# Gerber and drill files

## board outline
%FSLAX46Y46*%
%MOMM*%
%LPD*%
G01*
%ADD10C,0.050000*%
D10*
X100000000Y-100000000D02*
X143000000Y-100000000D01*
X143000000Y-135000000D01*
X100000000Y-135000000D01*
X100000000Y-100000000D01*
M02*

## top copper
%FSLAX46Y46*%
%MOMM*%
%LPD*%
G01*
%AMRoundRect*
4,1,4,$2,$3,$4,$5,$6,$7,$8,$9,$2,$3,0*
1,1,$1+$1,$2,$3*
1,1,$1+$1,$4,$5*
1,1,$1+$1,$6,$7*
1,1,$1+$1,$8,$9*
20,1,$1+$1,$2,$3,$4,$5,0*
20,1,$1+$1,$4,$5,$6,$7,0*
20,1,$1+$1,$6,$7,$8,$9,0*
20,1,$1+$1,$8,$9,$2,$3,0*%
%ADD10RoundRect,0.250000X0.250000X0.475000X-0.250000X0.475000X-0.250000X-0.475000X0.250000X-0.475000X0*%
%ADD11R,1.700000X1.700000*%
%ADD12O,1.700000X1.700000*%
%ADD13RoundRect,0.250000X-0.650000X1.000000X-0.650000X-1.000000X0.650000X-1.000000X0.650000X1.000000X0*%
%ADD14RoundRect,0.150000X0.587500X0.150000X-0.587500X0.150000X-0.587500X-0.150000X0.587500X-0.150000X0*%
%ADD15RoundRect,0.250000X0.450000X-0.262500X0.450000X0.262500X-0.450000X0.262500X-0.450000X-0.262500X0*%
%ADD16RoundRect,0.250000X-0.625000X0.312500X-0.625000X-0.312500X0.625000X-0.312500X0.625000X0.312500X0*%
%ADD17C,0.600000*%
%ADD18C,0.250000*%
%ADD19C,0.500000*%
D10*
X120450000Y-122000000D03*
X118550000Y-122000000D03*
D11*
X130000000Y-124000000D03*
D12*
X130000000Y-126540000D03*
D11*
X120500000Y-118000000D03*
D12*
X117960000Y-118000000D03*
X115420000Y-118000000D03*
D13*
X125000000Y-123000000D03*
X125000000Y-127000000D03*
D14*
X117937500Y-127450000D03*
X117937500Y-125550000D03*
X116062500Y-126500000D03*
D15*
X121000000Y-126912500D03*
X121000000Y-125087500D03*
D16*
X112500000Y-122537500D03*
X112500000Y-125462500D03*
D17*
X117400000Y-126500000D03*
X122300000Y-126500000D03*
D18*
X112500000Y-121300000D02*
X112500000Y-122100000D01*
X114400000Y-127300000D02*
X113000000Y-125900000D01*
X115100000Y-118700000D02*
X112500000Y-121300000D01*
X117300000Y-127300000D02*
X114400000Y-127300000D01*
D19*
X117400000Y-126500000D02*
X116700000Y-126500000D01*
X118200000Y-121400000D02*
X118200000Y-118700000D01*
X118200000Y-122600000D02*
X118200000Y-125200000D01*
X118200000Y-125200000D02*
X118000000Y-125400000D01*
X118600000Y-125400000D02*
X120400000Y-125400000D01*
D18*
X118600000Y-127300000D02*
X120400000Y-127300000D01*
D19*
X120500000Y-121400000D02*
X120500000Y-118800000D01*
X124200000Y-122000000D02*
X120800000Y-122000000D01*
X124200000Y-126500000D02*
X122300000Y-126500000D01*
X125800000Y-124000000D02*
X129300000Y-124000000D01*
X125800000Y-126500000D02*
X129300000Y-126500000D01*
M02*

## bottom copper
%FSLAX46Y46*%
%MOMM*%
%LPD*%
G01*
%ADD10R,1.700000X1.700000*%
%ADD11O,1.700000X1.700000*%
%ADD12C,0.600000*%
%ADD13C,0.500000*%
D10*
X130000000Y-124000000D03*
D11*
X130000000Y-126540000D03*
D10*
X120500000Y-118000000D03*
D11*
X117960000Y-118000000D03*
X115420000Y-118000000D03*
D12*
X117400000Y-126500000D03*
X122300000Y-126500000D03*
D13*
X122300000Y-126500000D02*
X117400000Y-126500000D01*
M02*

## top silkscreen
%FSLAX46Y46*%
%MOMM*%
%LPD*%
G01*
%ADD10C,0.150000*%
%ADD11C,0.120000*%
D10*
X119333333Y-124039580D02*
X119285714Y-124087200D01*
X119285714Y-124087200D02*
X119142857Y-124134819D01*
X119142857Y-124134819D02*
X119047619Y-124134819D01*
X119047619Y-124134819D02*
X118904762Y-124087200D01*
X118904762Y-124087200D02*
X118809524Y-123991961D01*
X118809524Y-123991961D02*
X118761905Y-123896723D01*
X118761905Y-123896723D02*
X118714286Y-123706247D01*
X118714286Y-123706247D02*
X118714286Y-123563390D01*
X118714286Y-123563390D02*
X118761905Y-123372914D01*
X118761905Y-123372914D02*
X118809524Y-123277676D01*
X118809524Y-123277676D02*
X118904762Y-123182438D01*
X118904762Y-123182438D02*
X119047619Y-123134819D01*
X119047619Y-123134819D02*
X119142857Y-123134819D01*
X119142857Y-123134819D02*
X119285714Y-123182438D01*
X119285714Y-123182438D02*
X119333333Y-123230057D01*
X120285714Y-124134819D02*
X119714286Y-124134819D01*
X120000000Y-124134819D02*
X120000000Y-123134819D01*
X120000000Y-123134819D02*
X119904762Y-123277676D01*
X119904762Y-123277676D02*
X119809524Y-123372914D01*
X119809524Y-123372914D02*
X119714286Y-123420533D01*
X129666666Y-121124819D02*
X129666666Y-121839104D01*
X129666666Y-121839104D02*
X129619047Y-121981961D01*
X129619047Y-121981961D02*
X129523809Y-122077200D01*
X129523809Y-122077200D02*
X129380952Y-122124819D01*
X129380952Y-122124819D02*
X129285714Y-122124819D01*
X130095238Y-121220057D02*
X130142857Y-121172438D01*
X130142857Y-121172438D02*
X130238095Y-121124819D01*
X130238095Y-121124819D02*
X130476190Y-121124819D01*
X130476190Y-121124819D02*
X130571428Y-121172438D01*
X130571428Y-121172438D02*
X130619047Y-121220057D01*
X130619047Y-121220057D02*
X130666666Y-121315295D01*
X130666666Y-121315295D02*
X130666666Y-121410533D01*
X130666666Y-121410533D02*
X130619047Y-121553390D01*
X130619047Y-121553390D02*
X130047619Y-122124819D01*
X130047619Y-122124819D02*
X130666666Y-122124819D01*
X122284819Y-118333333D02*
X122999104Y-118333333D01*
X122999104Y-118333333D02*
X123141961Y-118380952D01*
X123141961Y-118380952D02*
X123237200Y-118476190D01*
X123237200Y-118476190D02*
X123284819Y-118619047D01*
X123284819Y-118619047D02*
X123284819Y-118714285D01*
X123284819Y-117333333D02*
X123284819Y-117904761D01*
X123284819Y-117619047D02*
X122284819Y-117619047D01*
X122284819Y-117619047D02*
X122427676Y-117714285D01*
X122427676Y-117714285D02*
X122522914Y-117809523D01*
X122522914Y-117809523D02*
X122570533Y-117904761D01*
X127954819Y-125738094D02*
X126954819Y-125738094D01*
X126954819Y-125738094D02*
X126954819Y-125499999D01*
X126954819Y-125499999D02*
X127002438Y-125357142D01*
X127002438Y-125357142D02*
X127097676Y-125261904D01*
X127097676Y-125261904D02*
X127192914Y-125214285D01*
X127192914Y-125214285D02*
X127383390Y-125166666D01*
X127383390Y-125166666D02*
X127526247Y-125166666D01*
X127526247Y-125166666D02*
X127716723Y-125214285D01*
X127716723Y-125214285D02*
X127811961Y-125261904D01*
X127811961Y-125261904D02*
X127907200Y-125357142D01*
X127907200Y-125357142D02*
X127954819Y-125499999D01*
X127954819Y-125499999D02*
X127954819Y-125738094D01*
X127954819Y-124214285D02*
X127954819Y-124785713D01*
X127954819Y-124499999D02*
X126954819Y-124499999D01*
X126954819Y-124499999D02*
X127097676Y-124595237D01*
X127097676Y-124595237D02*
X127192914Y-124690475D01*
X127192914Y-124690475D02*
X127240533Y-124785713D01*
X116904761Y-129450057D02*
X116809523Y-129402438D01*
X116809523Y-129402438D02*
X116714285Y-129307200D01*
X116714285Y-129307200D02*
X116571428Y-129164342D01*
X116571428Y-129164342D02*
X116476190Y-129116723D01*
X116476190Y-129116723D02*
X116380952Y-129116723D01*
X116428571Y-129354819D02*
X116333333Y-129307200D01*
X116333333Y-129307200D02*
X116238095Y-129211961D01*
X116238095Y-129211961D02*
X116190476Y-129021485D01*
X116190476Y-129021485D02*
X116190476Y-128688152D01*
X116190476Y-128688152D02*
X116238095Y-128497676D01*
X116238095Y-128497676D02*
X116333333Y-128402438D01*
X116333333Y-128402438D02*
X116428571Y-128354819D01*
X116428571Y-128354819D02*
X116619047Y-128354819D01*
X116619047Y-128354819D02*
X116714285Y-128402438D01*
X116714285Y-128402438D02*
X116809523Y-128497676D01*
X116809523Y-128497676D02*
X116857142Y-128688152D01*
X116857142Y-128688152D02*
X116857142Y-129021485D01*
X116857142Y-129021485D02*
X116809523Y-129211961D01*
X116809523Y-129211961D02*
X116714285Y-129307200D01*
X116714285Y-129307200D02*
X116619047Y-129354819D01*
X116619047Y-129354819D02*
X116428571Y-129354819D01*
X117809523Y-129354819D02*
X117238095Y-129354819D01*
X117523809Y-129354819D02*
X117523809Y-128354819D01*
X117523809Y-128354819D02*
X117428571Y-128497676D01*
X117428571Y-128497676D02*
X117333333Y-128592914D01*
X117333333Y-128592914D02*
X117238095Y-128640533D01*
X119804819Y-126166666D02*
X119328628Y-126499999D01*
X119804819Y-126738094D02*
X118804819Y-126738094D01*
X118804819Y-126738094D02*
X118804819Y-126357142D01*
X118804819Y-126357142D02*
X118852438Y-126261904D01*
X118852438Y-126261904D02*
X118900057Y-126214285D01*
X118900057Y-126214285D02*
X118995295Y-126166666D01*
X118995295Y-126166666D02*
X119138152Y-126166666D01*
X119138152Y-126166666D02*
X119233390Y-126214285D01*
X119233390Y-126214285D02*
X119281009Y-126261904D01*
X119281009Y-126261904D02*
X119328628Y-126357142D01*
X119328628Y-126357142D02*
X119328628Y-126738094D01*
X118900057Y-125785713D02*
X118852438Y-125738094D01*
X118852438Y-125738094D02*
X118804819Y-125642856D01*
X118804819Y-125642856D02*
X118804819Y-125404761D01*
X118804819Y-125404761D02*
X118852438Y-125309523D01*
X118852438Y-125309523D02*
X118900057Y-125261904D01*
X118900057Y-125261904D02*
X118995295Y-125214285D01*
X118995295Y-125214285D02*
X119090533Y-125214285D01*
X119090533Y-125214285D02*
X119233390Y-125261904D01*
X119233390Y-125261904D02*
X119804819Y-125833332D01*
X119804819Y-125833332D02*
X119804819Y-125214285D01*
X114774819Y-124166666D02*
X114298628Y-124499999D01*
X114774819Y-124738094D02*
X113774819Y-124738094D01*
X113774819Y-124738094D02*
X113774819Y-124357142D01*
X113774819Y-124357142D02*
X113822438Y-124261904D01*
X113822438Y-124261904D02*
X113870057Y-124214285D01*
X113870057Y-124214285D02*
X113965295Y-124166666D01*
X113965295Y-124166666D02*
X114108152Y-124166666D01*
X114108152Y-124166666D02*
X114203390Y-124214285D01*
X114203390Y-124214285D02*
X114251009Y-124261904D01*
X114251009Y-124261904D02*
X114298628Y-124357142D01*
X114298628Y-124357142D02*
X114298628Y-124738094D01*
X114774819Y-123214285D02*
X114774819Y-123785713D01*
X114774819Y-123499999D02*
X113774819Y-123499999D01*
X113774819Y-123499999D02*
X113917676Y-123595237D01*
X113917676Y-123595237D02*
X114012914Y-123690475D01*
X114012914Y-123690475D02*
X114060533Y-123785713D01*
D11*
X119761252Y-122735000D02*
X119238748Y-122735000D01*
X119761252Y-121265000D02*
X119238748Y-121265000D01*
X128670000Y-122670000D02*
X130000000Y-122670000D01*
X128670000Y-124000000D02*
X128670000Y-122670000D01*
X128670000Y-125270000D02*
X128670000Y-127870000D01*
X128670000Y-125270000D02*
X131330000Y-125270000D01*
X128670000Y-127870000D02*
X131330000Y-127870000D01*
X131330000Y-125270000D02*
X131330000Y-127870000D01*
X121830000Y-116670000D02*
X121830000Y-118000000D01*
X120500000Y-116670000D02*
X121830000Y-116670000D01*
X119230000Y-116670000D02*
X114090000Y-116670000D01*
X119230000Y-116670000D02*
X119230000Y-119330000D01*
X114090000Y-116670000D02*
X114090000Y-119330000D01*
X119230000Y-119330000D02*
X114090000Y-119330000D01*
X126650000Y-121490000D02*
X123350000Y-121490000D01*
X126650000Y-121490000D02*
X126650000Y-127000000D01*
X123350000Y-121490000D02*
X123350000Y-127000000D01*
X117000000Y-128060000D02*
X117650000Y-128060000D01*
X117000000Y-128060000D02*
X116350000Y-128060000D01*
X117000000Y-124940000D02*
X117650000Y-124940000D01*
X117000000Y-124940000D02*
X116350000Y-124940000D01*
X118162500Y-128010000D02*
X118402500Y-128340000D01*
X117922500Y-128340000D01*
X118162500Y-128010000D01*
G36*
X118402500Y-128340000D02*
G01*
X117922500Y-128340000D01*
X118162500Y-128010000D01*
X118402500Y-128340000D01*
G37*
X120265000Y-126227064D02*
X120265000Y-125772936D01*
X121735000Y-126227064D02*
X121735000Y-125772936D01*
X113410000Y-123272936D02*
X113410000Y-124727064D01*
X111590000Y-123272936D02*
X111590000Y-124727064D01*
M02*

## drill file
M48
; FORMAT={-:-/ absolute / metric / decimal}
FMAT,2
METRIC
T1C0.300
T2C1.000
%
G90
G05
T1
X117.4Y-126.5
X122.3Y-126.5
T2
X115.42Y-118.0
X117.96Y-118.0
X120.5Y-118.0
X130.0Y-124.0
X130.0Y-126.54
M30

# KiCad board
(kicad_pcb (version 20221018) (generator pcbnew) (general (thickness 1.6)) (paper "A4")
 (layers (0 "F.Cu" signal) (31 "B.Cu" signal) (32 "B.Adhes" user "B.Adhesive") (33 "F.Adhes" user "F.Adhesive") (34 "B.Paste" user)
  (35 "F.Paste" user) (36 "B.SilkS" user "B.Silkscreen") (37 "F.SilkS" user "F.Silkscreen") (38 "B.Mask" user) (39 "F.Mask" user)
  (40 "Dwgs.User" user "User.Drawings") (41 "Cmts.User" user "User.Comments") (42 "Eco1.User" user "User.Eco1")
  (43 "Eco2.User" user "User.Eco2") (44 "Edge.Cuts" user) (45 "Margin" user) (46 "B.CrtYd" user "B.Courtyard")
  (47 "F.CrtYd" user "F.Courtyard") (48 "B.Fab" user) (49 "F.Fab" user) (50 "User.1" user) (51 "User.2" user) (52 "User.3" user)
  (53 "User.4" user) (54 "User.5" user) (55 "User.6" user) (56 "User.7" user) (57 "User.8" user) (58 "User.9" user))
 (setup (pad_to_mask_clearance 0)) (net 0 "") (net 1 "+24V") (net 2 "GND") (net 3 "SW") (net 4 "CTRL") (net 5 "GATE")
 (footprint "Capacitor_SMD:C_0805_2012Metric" (layer "F.Cu") (at 119.5 122 180)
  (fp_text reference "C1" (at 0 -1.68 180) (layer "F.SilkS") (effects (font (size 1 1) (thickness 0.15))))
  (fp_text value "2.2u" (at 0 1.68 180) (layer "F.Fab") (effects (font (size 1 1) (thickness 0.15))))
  (fp_line (start -0.261252 -0.735) (end 0.261252 -0.735) (stroke (width 0.12) (type solid)) (layer "F.SilkS"))
  (fp_line (start -0.261252 0.735) (end 0.261252 0.735) (stroke (width 0.12) (type solid)) (layer "F.SilkS"))
  (pad "1" smd roundrect (at -0.95 0 180) (size 1 1.45) (layers "F.Cu" "F.Paste" "F.Mask") (roundrect_rratio 0.25) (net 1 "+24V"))
  (pad "2" smd roundrect (at 0.95 0 180) (size 1 1.45) (layers "F.Cu" "F.Paste" "F.Mask") (roundrect_rratio 0.25) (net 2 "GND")))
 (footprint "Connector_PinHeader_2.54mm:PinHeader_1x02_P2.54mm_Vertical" (layer "F.Cu") (at 130 124)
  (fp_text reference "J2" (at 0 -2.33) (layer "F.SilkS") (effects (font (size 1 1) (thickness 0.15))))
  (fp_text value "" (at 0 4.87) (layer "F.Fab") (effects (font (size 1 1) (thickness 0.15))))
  (fp_line (start -1.33 -1.33) (end 0 -1.33) (stroke (width 0.12) (type solid)) (layer "F.SilkS"))
  (fp_line (start -1.33 0) (end -1.33 -1.33) (stroke (width 0.12) (type solid)) (layer "F.SilkS"))
  (fp_line (start -1.33 1.27) (end -1.33 3.87) (stroke (width 0.12) (type solid)) (layer "F.SilkS"))
  (fp_line (start -1.33 1.27) (end 1.33 1.27) (stroke (width 0.12) (type solid)) (layer "F.SilkS"))
  (fp_line (start -1.33 3.87) (end 1.33 3.87) (stroke (width 0.12) (type solid)) (layer "F.SilkS"))
  (fp_line (start 1.33 1.27) (end 1.33 3.87) (stroke (width 0.12) (type solid)) (layer "F.SilkS"))
  (pad "1" thru_hole rect (at 0 0) (size 1.7 1.7) (drill 1) (layers "*.Cu" "*.Mask") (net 1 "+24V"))
  (pad "2" thru_hole oval (at 0 2.54) (size 1.7 1.7) (drill 1) (layers "*.Cu" "*.Mask") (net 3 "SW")))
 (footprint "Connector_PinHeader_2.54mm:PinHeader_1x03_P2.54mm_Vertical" (layer "F.Cu") (at 120.5 118 -90)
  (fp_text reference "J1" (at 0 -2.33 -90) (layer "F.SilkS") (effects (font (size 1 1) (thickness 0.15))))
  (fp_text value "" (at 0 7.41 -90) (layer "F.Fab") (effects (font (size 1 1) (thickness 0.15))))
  (fp_line (start -1.33 -1.33) (end 0 -1.33) (stroke (width 0.12) (type solid)) (layer "F.SilkS"))
  (fp_line (start -1.33 0) (end -1.33 -1.33) (stroke (width 0.12) (type solid)) (layer "F.SilkS"))
  (fp_line (start -1.33 1.27) (end -1.33 6.41) (stroke (width 0.12) (type solid)) (layer "F.SilkS"))
  (fp_line (start -1.33 1.27) (end 1.33 1.27) (stroke (width 0.12) (type solid)) (layer "F.SilkS"))
  (fp_line (start -1.33 6.41) (end 1.33 6.41) (stroke (width 0.12) (type solid)) (layer "F.SilkS"))
  (fp_line (start 1.33 1.27) (end 1.33 6.41) (stroke (width 0.12) (type solid)) (layer "F.SilkS"))
  (pad "1" thru_hole rect (at 0 0 270) (size 1.7 1.7) (drill 1) (layers "*.Cu" "*.Mask") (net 1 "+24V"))
  (pad "2" thru_hole oval (at 0 2.54 270) (size 1.7 1.7) (drill 1) (layers "*.Cu" "*.Mask") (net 2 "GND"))
  (pad "3" thru_hole oval (at 0 5.08 270) (size 1.7 1.7) (drill 1) (layers "*.Cu" "*.Mask") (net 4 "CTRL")))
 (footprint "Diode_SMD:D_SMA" (layer "F.Cu") (at 125 125 -90)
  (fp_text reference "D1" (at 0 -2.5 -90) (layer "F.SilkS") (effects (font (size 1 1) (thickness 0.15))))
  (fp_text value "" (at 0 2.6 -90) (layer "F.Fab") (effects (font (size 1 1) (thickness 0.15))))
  (fp_line (start -3.51 -1.65) (end -3.51 1.65) (stroke (width 0.12) (type solid)) (layer "F.SilkS"))
  (fp_line (start -3.51 -1.65) (end 2 -1.65) (stroke (width 0.12) (type solid)) (layer "F.SilkS"))
  (fp_line (start -3.51 1.65) (end 2 1.65) (stroke (width 0.12) (type solid)) (layer "F.SilkS"))
  (pad "1" smd roundrect (at -2 0 270) (size 2.5 1.8) (layers "F.Cu" "F.Paste" "F.Mask") (roundrect_rratio 0.1388888889) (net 1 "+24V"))
  (pad "2" smd roundrect (at 2 0 270) (size 2.5 1.8) (layers "F.Cu" "F.Paste" "F.Mask") (roundrect_rratio 0.1388888889) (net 3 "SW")))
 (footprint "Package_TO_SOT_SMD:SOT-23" (layer "F.Cu") (at 117 126.5 180)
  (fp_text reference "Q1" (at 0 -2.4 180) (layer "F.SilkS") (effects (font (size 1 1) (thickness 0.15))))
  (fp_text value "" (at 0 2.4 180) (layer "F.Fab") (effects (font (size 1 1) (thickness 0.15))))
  (fp_line (start 0 -1.56) (end -0.65 -1.56) (stroke (width 0.12) (type solid)) (layer "F.SilkS"))
  (fp_line (start 0 -1.56) (end 0.65 -1.56) (stroke (width 0.12) (type solid)) (layer "F.SilkS"))
  (fp_line (start 0 1.56) (end -0.65 1.56) (stroke (width 0.12) (type solid)) (layer "F.SilkS"))
  (fp_line (start 0 1.56) (end 0.65 1.56) (stroke (width 0.12) (type solid)) (layer "F.SilkS"))
  (fp_poly
   (pts (xy -1.1625 -1.51) (xy -1.4025 -1.84) (xy -0.9225 -1.84) (xy -1.1625 -1.51)) (stroke (width 0.12) (type solid)) (fill solid)
   (layer "F.SilkS"))
  (pad "1" smd roundrect (at -0.9375 -0.95 180) (size 1.475 0.6) (layers "F.Cu" "F.Paste" "F.Mask") (roundrect_rratio 0.25) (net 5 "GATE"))
  (pad "2" smd roundrect (at -0.9375 0.95 180) (size 1.475 0.6) (layers "F.Cu" "F.Paste" "F.Mask") (roundrect_rratio 0.25) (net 2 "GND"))
  (pad "3" smd roundrect (at 0.9375 0 180) (size 1.475 0.6) (layers "F.Cu" "F.Paste" "F.Mask") (roundrect_rratio 0.25) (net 3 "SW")))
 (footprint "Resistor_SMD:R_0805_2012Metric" (layer "F.Cu") (at 121 126 90)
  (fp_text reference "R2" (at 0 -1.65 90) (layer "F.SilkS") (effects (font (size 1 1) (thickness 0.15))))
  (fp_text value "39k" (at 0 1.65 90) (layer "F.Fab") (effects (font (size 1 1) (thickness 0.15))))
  (fp_line (start -0.227064 -0.735) (end 0.227064 -0.735) (stroke (width 0.12) (type solid)) (layer "F.SilkS"))
  (fp_line (start -0.227064 0.735) (end 0.227064 0.735) (stroke (width 0.12) (type solid)) (layer "F.SilkS"))
  (pad "1" smd roundrect (at -0.9125 0 90) (size 1.025 1.4) (layers "F.Cu" "F.Paste" "F.Mask") (roundrect_rratio 0.243902) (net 5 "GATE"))
  (pad "2" smd roundrect (at 0.9125 0 90) (size 1.025 1.4) (layers "F.Cu" "F.Paste" "F.Mask") (roundrect_rratio 0.243902) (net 2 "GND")))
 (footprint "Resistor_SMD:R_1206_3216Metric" (layer "F.Cu") (at 112.5 124 -90)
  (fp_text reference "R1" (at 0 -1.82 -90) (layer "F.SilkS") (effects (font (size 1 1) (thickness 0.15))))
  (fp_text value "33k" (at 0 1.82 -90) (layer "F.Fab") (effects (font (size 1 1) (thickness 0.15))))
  (fp_line (start -0.727064 -0.91) (end 0.727064 -0.91) (stroke (width 0.12) (type solid)) (layer "F.SilkS"))
  (fp_line (start -0.727064 0.91) (end 0.727064 0.91) (stroke (width 0.12) (type solid)) (layer "F.SilkS"))
  (pad "1" smd roundrect (at -1.4625 0 270) (size 1.125 1.75) (layers "F.Cu" "F.Paste" "F.Mask") (roundrect_rratio 0.222222) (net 4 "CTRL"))
  (pad "2" smd roundrect (at 1.4625 0 270) (size 1.125 1.75) (layers "F.Cu" "F.Paste" "F.Mask") (roundrect_rratio 0.222222) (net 5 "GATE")))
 (gr_rect (start 100 100) (end 143 135) (stroke (width 0.05) (type default)) (fill none) (layer "Edge.Cuts"))
 (segment (start 112.5 121.3) (end 112.5 122.1) (width 0.25) (layer "F.Cu") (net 4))
 (segment (start 114.4 127.3) (end 113 125.9) (width 0.25) (layer "F.Cu") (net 5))
 (segment (start 115.1 118.7) (end 112.5 121.3) (width 0.25) (layer "F.Cu") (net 4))
 (segment (start 117.3 127.3) (end 114.4 127.3) (width 0.25) (layer "F.Cu") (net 5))
 (segment (start 117.4 126.5) (end 116.7 126.5) (width 0.5) (layer "F.Cu") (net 3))
 (segment (start 118.2 121.4) (end 118.2 118.7) (width 0.5) (layer "F.Cu") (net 2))
 (segment (start 118.2 122.6) (end 118.2 125.2) (width 0.5) (layer "F.Cu") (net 2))
 (segment (start 118.2 125.2) (end 118 125.4) (width 0.5) (layer "F.Cu") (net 2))
 (segment (start 118.6 125.4) (end 120.4 125.4) (width 0.5) (layer "F.Cu") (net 2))
 (segment (start 118.6 127.3) (end 120.4 127.3) (width 0.25) (layer "F.Cu") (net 5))
 (segment (start 120.5 121.4) (end 120.5 118.8) (width 0.5) (layer "F.Cu") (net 1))
 (segment (start 124.2 122) (end 120.8 122) (width 0.5) (layer "F.Cu") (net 1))
 (segment (start 124.2 126.5) (end 122.3 126.5) (width 0.5) (layer "F.Cu") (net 3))
 (segment (start 125.8 124) (end 129.3 124) (width 0.5) (layer "F.Cu") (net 1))
 (segment (start 125.8 126.5) (end 129.3 126.5) (width 0.5) (layer "F.Cu") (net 3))
 (via (at 117.4 126.5) (size 0.6) (drill 0.3) (layers "F.Cu" "B.Cu") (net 3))
 (via (at 122.3 126.5) (size 0.6) (drill 0.3) (layers "F.Cu" "B.Cu") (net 3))
 (segment (start 122.3 126.5) (end 117.4 126.5) (width 0.5) (layer "B.Cu") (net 3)))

